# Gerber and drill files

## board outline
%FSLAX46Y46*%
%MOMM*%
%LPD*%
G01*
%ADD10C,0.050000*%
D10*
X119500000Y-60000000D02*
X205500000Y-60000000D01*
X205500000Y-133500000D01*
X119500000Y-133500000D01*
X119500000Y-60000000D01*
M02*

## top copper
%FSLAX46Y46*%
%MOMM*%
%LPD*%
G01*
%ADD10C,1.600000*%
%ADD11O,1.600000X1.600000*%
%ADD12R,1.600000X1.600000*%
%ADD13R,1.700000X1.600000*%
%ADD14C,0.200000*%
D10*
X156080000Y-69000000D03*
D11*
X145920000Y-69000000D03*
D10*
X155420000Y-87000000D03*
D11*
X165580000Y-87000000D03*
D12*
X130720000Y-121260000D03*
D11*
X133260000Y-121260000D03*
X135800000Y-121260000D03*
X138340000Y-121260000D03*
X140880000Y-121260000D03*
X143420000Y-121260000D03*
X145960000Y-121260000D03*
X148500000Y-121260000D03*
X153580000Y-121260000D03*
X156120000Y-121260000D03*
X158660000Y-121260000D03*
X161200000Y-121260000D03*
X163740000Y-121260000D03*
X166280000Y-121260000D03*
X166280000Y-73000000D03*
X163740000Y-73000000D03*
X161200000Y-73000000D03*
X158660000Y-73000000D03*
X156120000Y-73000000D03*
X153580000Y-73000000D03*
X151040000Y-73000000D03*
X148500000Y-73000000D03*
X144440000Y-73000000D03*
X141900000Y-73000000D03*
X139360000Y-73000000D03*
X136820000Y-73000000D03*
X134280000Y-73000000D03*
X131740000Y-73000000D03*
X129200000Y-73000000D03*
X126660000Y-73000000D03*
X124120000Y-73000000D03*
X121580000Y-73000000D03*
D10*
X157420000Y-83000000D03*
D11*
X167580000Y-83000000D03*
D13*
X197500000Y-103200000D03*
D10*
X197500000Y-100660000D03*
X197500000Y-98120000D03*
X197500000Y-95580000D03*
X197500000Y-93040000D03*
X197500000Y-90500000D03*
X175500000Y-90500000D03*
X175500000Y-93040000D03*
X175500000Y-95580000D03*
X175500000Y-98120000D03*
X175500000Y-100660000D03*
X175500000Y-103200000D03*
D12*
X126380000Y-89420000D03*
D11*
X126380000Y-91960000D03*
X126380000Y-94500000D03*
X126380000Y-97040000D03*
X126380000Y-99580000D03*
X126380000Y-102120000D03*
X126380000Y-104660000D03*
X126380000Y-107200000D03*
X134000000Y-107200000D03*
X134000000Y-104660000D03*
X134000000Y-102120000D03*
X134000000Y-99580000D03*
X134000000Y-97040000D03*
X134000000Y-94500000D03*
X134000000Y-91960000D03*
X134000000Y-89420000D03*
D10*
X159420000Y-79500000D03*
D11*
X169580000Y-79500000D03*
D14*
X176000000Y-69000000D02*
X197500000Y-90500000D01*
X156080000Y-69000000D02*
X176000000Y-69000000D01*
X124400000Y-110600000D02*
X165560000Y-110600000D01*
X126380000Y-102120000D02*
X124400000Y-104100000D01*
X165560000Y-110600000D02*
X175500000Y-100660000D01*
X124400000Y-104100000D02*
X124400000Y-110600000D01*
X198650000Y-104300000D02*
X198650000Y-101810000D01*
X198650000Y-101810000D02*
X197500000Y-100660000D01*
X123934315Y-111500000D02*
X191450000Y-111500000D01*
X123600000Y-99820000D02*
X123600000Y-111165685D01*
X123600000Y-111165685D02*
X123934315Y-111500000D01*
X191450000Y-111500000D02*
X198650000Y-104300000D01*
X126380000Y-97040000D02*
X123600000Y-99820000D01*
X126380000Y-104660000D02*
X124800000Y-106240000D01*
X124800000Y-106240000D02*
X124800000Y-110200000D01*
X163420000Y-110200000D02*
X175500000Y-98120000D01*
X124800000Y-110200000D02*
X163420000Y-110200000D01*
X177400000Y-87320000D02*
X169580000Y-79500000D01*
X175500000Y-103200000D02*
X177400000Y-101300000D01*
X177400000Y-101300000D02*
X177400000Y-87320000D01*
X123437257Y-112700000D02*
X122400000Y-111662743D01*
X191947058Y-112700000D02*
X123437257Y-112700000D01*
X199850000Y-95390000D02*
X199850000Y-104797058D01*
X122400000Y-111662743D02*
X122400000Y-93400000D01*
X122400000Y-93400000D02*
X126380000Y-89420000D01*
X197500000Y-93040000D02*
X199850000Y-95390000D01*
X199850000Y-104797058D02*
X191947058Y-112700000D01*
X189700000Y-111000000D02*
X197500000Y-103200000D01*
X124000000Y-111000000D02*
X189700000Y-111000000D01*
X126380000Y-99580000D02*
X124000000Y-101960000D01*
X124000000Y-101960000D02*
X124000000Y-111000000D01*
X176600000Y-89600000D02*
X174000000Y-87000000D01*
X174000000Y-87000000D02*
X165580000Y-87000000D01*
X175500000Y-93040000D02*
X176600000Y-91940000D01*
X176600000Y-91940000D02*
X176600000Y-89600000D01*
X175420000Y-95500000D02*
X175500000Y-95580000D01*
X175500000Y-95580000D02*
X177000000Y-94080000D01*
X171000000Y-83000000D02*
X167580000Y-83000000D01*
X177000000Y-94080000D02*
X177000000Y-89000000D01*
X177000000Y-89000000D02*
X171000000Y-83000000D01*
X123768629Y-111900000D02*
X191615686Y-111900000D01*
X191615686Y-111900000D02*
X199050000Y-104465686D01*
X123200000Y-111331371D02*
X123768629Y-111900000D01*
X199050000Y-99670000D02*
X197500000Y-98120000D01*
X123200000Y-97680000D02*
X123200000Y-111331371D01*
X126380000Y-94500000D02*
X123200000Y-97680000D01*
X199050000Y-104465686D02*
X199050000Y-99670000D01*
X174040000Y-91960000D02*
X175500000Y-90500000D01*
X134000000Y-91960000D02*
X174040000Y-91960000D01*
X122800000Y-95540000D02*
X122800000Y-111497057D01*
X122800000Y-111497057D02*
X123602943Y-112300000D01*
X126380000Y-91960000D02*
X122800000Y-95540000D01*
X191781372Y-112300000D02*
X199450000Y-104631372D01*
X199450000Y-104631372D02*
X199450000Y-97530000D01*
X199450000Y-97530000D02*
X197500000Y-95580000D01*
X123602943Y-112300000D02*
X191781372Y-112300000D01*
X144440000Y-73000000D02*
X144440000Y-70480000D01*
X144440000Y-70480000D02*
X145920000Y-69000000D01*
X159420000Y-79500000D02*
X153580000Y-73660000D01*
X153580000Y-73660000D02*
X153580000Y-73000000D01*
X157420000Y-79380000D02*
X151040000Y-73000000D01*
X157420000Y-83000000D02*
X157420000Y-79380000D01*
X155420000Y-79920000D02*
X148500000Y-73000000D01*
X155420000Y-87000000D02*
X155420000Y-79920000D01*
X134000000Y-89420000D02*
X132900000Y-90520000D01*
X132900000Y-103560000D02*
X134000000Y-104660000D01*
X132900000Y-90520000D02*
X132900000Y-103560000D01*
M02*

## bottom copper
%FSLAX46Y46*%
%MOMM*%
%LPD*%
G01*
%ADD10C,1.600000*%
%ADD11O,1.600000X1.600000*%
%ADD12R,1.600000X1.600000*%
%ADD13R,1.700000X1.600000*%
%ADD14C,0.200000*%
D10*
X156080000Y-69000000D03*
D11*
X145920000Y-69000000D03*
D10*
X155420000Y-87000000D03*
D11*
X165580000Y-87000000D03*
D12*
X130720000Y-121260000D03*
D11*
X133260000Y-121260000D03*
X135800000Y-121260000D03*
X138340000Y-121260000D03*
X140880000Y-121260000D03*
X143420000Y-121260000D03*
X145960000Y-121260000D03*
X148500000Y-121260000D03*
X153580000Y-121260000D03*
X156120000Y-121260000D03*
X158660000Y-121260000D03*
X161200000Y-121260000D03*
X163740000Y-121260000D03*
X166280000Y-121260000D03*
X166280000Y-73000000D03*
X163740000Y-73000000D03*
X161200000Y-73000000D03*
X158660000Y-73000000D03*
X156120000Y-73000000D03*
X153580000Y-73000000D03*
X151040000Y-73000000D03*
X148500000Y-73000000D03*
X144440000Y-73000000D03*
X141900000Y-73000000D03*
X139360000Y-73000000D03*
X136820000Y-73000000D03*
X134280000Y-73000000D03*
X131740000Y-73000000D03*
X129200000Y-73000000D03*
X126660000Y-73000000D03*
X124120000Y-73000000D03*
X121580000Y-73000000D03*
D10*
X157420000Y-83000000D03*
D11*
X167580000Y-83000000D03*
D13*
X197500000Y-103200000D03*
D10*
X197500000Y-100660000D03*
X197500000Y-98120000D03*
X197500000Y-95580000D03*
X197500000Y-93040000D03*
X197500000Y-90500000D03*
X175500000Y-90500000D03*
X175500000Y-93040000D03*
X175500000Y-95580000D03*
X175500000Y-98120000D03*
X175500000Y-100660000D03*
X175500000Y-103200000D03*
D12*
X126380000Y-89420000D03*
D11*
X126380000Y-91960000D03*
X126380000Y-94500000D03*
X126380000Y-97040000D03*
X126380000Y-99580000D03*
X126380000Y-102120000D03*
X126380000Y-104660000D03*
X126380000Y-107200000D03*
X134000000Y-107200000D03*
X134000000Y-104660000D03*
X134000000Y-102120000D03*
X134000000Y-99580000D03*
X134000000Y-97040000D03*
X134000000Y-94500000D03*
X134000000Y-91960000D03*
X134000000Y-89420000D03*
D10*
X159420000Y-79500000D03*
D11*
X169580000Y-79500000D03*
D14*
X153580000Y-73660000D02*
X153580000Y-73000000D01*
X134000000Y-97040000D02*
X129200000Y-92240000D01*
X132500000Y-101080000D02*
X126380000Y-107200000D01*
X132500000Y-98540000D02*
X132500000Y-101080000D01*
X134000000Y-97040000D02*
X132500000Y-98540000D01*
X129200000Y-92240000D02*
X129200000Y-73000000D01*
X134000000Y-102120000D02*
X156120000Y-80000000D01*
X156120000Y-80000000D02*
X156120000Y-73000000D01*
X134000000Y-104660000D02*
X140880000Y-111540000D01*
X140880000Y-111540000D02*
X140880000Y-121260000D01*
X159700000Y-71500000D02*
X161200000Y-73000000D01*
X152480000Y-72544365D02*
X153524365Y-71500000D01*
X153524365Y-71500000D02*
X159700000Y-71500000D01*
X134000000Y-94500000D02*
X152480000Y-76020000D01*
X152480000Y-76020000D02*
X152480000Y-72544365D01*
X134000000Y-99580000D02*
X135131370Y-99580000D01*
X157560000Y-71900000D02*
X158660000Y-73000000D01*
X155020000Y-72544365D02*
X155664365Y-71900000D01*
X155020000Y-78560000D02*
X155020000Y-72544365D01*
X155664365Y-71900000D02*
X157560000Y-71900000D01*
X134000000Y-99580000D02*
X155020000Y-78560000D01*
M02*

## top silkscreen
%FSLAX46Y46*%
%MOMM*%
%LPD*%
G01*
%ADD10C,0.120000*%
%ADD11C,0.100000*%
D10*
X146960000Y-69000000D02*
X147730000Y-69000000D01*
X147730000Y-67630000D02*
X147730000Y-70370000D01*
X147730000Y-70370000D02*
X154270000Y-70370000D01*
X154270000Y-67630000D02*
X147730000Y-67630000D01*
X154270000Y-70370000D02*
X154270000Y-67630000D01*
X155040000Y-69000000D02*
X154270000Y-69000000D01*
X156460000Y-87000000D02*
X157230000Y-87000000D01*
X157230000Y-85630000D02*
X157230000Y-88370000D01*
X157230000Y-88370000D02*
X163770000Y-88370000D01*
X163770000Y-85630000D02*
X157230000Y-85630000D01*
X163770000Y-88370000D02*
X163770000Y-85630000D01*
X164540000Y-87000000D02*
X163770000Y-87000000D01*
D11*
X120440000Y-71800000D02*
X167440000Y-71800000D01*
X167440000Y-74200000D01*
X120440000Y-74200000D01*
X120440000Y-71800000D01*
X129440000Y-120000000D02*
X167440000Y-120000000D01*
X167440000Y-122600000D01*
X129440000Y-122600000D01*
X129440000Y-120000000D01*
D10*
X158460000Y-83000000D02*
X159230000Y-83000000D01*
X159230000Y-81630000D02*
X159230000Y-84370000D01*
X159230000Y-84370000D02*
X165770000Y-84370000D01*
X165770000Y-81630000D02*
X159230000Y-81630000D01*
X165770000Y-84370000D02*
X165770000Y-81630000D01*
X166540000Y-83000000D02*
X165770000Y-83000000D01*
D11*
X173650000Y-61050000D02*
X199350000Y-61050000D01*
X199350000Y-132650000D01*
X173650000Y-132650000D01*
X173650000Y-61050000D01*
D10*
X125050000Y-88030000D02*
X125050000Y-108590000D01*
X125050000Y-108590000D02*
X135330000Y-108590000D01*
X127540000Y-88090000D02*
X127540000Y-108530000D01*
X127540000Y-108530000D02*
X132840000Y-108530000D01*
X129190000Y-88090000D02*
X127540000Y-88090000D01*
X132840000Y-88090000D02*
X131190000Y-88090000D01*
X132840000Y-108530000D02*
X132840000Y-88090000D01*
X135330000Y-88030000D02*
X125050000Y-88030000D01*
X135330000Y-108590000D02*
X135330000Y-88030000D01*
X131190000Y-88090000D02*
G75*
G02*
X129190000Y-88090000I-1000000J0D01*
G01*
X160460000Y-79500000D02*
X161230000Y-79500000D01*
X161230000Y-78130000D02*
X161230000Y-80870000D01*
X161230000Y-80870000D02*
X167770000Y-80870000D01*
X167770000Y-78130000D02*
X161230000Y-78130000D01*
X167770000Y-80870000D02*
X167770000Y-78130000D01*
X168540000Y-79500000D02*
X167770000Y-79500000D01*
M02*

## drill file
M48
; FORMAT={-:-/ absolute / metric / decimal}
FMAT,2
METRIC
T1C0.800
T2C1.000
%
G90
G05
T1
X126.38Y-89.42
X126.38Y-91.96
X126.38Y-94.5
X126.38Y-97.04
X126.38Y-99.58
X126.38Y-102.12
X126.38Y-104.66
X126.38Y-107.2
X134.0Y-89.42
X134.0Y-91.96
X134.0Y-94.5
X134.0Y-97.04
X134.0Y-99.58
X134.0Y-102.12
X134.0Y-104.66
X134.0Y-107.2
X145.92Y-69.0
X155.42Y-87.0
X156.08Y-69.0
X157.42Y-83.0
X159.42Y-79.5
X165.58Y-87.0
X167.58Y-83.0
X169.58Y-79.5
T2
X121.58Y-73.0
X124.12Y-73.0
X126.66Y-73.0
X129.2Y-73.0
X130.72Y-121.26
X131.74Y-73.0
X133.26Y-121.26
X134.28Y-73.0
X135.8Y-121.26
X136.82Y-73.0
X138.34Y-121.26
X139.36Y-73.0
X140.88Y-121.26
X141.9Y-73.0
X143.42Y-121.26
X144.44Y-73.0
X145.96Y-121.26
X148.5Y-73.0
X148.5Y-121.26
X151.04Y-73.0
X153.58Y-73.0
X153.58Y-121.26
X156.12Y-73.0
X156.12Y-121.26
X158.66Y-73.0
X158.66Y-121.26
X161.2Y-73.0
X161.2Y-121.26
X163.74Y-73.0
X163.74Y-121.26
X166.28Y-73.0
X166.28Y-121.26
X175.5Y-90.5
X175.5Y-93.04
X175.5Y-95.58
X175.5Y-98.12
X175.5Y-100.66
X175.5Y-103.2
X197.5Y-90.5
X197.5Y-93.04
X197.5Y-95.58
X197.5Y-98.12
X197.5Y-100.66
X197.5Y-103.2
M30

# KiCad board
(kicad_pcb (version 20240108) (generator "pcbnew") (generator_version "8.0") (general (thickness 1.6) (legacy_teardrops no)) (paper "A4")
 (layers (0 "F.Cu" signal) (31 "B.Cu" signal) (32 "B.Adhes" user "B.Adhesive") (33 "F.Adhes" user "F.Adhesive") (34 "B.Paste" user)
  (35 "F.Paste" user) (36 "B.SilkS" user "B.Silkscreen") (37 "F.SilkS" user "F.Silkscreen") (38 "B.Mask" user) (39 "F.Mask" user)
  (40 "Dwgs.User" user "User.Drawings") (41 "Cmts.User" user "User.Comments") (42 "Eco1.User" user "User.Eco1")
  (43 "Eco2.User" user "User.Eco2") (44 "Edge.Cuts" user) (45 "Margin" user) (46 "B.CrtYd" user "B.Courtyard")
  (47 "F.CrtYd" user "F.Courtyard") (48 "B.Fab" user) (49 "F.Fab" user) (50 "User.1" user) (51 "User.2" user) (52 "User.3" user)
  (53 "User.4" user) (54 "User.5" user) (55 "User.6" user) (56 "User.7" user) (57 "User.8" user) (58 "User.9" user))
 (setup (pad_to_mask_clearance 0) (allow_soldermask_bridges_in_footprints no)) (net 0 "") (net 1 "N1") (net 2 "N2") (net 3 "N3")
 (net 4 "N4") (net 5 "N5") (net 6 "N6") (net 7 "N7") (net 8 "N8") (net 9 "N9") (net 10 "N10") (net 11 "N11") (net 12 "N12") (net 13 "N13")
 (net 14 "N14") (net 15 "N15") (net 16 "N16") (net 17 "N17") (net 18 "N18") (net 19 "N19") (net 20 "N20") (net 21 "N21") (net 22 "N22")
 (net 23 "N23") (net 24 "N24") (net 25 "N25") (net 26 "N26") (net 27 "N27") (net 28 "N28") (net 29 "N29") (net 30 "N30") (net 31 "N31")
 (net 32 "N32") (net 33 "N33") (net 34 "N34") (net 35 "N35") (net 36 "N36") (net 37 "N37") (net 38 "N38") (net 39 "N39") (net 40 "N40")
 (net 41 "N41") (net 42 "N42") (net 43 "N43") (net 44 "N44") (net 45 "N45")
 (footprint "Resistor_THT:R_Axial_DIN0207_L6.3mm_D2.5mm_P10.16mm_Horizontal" (layer "F.Cu") (at 156.08 69 180)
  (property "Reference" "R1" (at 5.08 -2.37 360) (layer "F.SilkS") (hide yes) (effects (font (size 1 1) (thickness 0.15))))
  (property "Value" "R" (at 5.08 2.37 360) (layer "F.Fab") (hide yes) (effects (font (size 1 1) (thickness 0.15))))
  (fp_line (start 9.12 0) (end 8.35 0) (stroke (width 0.12) (type solid)) (layer "F.SilkS"))
  (fp_line (start 8.35 1.37) (end 8.35 -1.37) (stroke (width 0.12) (type solid)) (layer "F.SilkS"))
  (fp_line (start 8.35 -1.37) (end 1.81 -1.37) (stroke (width 0.12) (type solid)) (layer "F.SilkS"))
  (fp_line (start 1.81 1.37) (end 8.35 1.37) (stroke (width 0.12) (type solid)) (layer "F.SilkS"))
  (fp_line (start 1.81 -1.37) (end 1.81 1.37) (stroke (width 0.12) (type solid)) (layer "F.SilkS"))
  (fp_line (start 1.04 0) (end 1.81 0) (stroke (width 0.12) (type solid)) (layer "F.SilkS"))
  (pad "1" thru_hole circle (at 0 0 180) (size 1.6 1.6) (drill 0.8) (layers "*.Cu" "*.Mask") (remove_unused_layers no) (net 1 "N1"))
  (pad "2" thru_hole oval (at 10.16 0 180) (size 1.6 1.6) (drill 0.8) (layers "*.Cu" "*.Mask") (remove_unused_layers no) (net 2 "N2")))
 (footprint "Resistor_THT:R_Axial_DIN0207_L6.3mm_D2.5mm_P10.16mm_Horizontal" (layer "F.Cu") (at 155.42 87)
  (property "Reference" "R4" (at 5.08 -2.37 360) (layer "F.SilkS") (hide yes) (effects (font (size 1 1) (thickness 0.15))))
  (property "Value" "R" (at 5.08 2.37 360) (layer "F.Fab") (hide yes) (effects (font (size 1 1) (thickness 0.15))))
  (fp_line (start 1.04 0) (end 1.81 0) (stroke (width 0.12) (type solid)) (layer "F.SilkS"))
  (fp_line (start 1.81 -1.37) (end 1.81 1.37) (stroke (width 0.12) (type solid)) (layer "F.SilkS"))
  (fp_line (start 1.81 1.37) (end 8.35 1.37) (stroke (width 0.12) (type solid)) (layer "F.SilkS"))
  (fp_line (start 8.35 -1.37) (end 1.81 -1.37) (stroke (width 0.12) (type solid)) (layer "F.SilkS"))
  (fp_line (start 8.35 1.37) (end 8.35 -1.37) (stroke (width 0.12) (type solid)) (layer "F.SilkS"))
  (fp_line (start 9.12 0) (end 8.35 0) (stroke (width 0.12) (type solid)) (layer "F.SilkS"))
  (pad "1" thru_hole circle (at 0 0) (size 1.6 1.6) (drill 0.8) (layers "*.Cu" "*.Mask") (remove_unused_layers no) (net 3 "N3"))
  (pad "2" thru_hole oval (at 10.16 0) (size 1.6 1.6) (drill 0.8) (layers "*.Cu" "*.Mask") (remove_unused_layers no) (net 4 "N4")))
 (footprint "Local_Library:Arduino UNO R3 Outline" (layer "F.Cu") (at 109.84 75.2)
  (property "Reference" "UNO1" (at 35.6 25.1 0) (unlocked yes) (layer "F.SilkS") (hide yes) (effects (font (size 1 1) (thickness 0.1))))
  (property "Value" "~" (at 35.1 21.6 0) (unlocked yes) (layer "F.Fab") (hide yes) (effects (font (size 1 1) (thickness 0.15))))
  (fp_rect (start 10.6 -3.4) (end 57.6 -1) (stroke (width 0.1) (type default)) (fill none) (layer "F.SilkS"))
  (fp_rect (start 19.6 44.8) (end 57.6 47.4) (stroke (width 0.1) (type default)) (fill none) (layer "F.SilkS"))
  (pad "1" thru_hole rect (at 20.88 46.06 90) (size 1.6 1.6) (drill 1) (layers "*.Cu" "*.Mask") (remove_unused_layers no) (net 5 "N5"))
  (pad "2" thru_hole oval (at 23.42 46.06 90) (size 1.6 1.6) (drill 1) (layers "*.Cu" "*.Mask") (remove_unused_layers no) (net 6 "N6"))
  (pad "3" thru_hole oval (at 25.96 46.06 90) (size 1.6 1.6) (drill 1) (layers "*.Cu" "*.Mask") (remove_unused_layers no) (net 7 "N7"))
  (pad "4" thru_hole oval (at 28.5 46.06 90) (size 1.6 1.6) (drill 1) (layers "*.Cu" "*.Mask") (remove_unused_layers no) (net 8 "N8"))
  (pad "5" thru_hole oval (at 31.04 46.06 90) (size 1.6 1.6) (drill 1) (layers "*.Cu" "*.Mask") (remove_unused_layers no) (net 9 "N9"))
  (pad "6" thru_hole oval (at 33.58 46.06 90) (size 1.6 1.6) (drill 1) (layers "*.Cu" "*.Mask") (remove_unused_layers no) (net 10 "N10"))
  (pad "7" thru_hole oval (at 36.12 46.06 90) (size 1.6 1.6) (drill 1) (layers "*.Cu" "*.Mask") (remove_unused_layers no) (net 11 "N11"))
  (pad "8" thru_hole oval (at 38.66 46.06 90) (size 1.6 1.6) (drill 1) (layers "*.Cu" "*.Mask") (remove_unused_layers no) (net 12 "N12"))
  (pad "9" thru_hole oval (at 43.74 46.06 90) (size 1.6 1.6) (drill 1) (layers "*.Cu" "*.Mask") (remove_unused_layers no) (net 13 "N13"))
  (pad "10" thru_hole oval (at 46.28 46.06 90) (size 1.6 1.6) (drill 1) (layers "*.Cu" "*.Mask") (remove_unused_layers no) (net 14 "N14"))
  (pad "11" thru_hole oval (at 48.82 46.06 90) (size 1.6 1.6) (drill 1) (layers "*.Cu" "*.Mask") (remove_unused_layers no) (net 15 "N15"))
  (pad "12" thru_hole oval (at 51.36 46.06 90) (size 1.6 1.6) (drill 1) (layers "*.Cu" "*.Mask") (remove_unused_layers no) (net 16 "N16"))
  (pad "13" thru_hole oval (at 53.9 46.06 90) (size 1.6 1.6) (drill 1) (layers "*.Cu" "*.Mask") (remove_unused_layers no) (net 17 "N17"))
  (pad "14" thru_hole oval (at 56.44 46.06 90) (size 1.6 1.6) (drill 1) (layers "*.Cu" "*.Mask") (remove_unused_layers no) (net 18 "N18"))
  (pad "15" thru_hole oval (at 56.44 -2.2 90) (size 1.6 1.6) (drill 1) (layers "*.Cu" "*.Mask") (remove_unused_layers no) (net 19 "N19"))
  (pad "16" thru_hole oval (at 53.9 -2.2 90) (size 1.6 1.6) (drill 1) (layers "*.Cu" "*.Mask") (remove_unused_layers no) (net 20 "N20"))
  (pad "17" thru_hole oval (at 51.36 -2.2 90) (size 1.6 1.6) (drill 1) (layers "*.Cu" "*.Mask") (remove_unused_layers no) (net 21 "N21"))
  (pad "18" thru_hole oval (at 48.82 -2.2 90) (size 1.6 1.6) (drill 1) (layers "*.Cu" "*.Mask") (remove_unused_layers no) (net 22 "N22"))
  (pad "19" thru_hole oval (at 46.28 -2.2 90) (size 1.6 1.6) (drill 1) (layers "*.Cu" "*.Mask") (remove_unused_layers no) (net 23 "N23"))
  (pad "20" thru_hole oval (at 43.74 -2.2 90) (size 1.6 1.6) (drill 1) (layers "*.Cu" "*.Mask") (remove_unused_layers no) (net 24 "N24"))
  (pad "21" thru_hole oval (at 41.2 -2.2 90) (size 1.6 1.6) (drill 1) (layers "*.Cu" "*.Mask") (remove_unused_layers no) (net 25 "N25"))
  (pad "22" thru_hole oval (at 38.66 -2.2 90) (size 1.6 1.6) (drill 1) (layers "*.Cu" "*.Mask") (remove_unused_layers no) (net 3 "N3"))
  (pad "23" thru_hole oval (at 34.6 -2.2 90) (size 1.6 1.6) (drill 1) (layers "*.Cu" "*.Mask") (remove_unused_layers no) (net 2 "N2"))
  (pad "24" thru_hole oval (at 32.06 -2.2 90) (size 1.6 1.6) (drill 1) (layers "*.Cu" "*.Mask") (remove_unused_layers no) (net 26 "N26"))
  (pad "25" thru_hole oval (at 29.52 -2.2 90) (size 1.6 1.6) (drill 1) (layers "*.Cu" "*.Mask") (remove_unused_layers no) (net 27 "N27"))
  (pad "26" thru_hole oval (at 26.98 -2.2 90) (size 1.6 1.6) (drill 1) (layers "*.Cu" "*.Mask") (remove_unused_layers no) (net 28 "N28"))
  (pad "27" thru_hole oval (at 24.44 -2.2 90) (size 1.6 1.6) (drill 1) (layers "*.Cu" "*.Mask") (remove_unused_layers no) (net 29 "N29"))
  (pad "28" thru_hole oval (at 21.9 -2.2 90) (size 1.6 1.6) (drill 1) (layers "*.Cu" "*.Mask") (remove_unused_layers no) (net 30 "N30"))
  (pad "29" thru_hole oval (at 19.36 -2.2 90) (size 1.6 1.6) (drill 1) (layers "*.Cu" "*.Mask") (remove_unused_layers no) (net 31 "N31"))
  (pad "30" thru_hole oval (at 16.82 -2.2 90) (size 1.6 1.6) (drill 1) (layers "*.Cu" "*.Mask") (remove_unused_layers no) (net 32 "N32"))
  (pad "31" thru_hole oval (at 14.28 -2.2 90) (size 1.6 1.6) (drill 1) (layers "*.Cu" "*.Mask") (remove_unused_layers no) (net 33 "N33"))
  (pad "32" thru_hole oval (at 11.74 -2.2 90) (size 1.6 1.6) (drill 1) (layers "*.Cu" "*.Mask") (remove_unused_layers no) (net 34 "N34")))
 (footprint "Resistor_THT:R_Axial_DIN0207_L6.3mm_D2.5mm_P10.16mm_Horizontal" (layer "F.Cu") (at 157.42 83)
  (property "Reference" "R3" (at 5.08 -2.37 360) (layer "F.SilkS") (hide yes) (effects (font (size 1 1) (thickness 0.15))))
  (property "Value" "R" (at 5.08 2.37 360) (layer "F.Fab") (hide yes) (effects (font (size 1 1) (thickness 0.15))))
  (fp_line (start 1.04 0) (end 1.81 0) (stroke (width 0.12) (type solid)) (layer "F.SilkS"))
  (fp_line (start 1.81 -1.37) (end 1.81 1.37) (stroke (width 0.12) (type solid)) (layer "F.SilkS"))
  (fp_line (start 1.81 1.37) (end 8.35 1.37) (stroke (width 0.12) (type solid)) (layer "F.SilkS"))
  (fp_line (start 8.35 -1.37) (end 1.81 -1.37) (stroke (width 0.12) (type solid)) (layer "F.SilkS"))
  (fp_line (start 8.35 1.37) (end 8.35 -1.37) (stroke (width 0.12) (type solid)) (layer "F.SilkS"))
  (fp_line (start 9.12 0) (end 8.35 0) (stroke (width 0.12) (type solid)) (layer "F.SilkS"))
  (pad "1" thru_hole circle (at 0 0) (size 1.6 1.6) (drill 0.8) (layers "*.Cu" "*.Mask") (remove_unused_layers no) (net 25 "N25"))
  (pad "2" thru_hole oval (at 10.16 0) (size 1.6 1.6) (drill 0.8) (layers "*.Cu" "*.Mask") (remove_unused_layers no) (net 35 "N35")))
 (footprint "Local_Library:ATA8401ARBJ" (layer "F.Cu") (at 186.5 96.85 90)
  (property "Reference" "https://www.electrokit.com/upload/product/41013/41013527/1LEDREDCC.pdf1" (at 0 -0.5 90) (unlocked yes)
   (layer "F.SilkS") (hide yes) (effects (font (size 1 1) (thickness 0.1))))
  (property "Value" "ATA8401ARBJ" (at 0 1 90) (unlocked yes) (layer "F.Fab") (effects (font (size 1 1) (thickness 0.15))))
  (fp_rect (start -35.8 -12.85) (end 35.8 12.85) (stroke (width 0.1) (type default)) (fill none) (layer "F.SilkS"))
  (pad "1" thru_hole rect (at -6.35 11 90) (size 1.6 1.7) (drill 1) (layers "*.Cu" "*.Mask") (remove_unused_layers no) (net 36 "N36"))
  (pad "2" thru_hole circle (at -3.81 11 90) (size 1.6 1.6) (drill 1) (layers "*.Cu" "*.Mask") (remove_unused_layers no) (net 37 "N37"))
  (pad "3" thru_hole circle (at -1.27 11 90) (size 1.6 1.6) (drill 1) (layers "*.Cu" "*.Mask") (remove_unused_layers no) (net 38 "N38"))
  (pad "4" thru_hole circle (at 1.27 11 90) (size 1.6 1.6) (drill 1) (layers "*.Cu" "*.Mask") (remove_unused_layers no) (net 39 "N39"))
  (pad "5" thru_hole circle (at 3.81 11 90) (size 1.6 1.6) (drill 1) (layers "*.Cu" "*.Mask") (remove_unused_layers no) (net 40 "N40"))
  (pad "6" thru_hole circle (at 6.35 11 90) (size 1.6 1.6) (drill 1) (layers "*.Cu" "*.Mask") (remove_unused_layers no) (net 1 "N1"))
  (pad "7" thru_hole circle (at 6.35 -11 270) (size 1.6 1.6) (drill 1) (layers "*.Cu" "*.Mask") (remove_unused_layers no) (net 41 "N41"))
  (pad "8" thru_hole circle (at 3.81 -11 270) (size 1.6 1.6) (drill 1) (layers "*.Cu" "*.Mask") (remove_unused_layers no) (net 4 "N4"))
  (pad "9" thru_hole circle (at 1.27 -11 270) (size 1.6 1.6) (drill 1) (layers "*.Cu" "*.Mask") (remove_unused_layers no) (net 35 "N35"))
  (pad "10" thru_hole circle (at -1.27 -11 270) (size 1.6 1.6) (drill 1) (layers "*.Cu" "*.Mask") (remove_unused_layers no) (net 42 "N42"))
  (pad "11" thru_hole circle (at -3.81 -11 270) (size 1.6 1.6) (drill 1) (layers "*.Cu" "*.Mask") (remove_unused_layers no) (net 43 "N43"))
  (pad "12" thru_hole circle (at -6.35 -11 270) (size 1.6 1.6) (drill 1) (layers "*.Cu" "*.Mask") (remove_unused_layers no) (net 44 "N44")))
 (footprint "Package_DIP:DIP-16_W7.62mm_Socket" (layer "F.Cu") (at 126.38 89.42)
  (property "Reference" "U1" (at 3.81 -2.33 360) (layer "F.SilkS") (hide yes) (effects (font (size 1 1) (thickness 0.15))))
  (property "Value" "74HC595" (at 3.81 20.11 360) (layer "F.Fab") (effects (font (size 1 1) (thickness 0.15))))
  (fp_line (start -1.33 -1.39) (end -1.33 19.17) (stroke (width 0.12) (type solid)) (layer "F.SilkS"))
  (fp_line (start -1.33 19.17) (end 8.95 19.17) (stroke (width 0.12) (type solid)) (layer "F.SilkS"))
  (fp_line (start 1.16 -1.33) (end 1.16 19.11) (stroke (width 0.12) (type solid)) (layer "F.SilkS"))
  (fp_line (start 1.16 19.11) (end 6.46 19.11) (stroke (width 0.12) (type solid)) (layer "F.SilkS"))
  (fp_line (start 2.81 -1.33) (end 1.16 -1.33) (stroke (width 0.12) (type solid)) (layer "F.SilkS"))
  (fp_line (start 6.46 -1.33) (end 4.81 -1.33) (stroke (width 0.12) (type solid)) (layer "F.SilkS"))
  (fp_line (start 6.46 19.11) (end 6.46 -1.33) (stroke (width 0.12) (type solid)) (layer "F.SilkS"))
  (fp_line (start 8.95 -1.39) (end -1.33 -1.39) (stroke (width 0.12) (type solid)) (layer "F.SilkS"))
  (fp_line (start 8.95 19.17) (end 8.95 -1.39) (stroke (width 0.12) (type solid)) (layer "F.SilkS"))
  (fp_arc (start 4.81 -1.33) (mid 3.81 -0.33) (end 2.81 -1.33) (stroke (width 0.12) (type solid)) (layer "F.SilkS"))
  (pad "1" thru_hole rect (at 0 0) (size 1.6 1.6) (drill 0.8) (layers "*.Cu" "*.Mask") (remove_unused_layers no) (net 40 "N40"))
  (pad "2" thru_hole oval (at 0 2.54) (size 1.6 1.6) (drill 0.8) (layers "*.Cu" "*.Mask") (remove_unused_layers no) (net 39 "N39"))
  (pad "3" thru_hole oval (at 0 5.08) (size 1.6 1.6) (drill 0.8) (layers "*.Cu" "*.Mask") (remove_unused_layers no) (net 38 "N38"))
  (pad "4" thru_hole oval (at 0 7.62) (size 1.6 1.6) (drill 0.8) (layers "*.Cu" "*.Mask") (remove_unused_layers no) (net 37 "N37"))
  (pad "5" thru_hole oval (at 0 10.16) (size 1.6 1.6) (drill 0.8) (layers "*.Cu" "*.Mask") (remove_unused_layers no) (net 36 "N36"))
  (pad "6" thru_hole oval (at 0 12.7) (size 1.6 1.6) (drill 0.8) (layers "*.Cu" "*.Mask") (remove_unused_layers no) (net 43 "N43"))
  (pad "7" thru_hole oval (at 0 15.24) (size 1.6 1.6) (drill 0.8) (layers "*.Cu" "*.Mask") (remove_unused_layers no) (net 42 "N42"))
  (pad "8" thru_hole oval (at 0 17.78) (size 1.6 1.6) (drill 0.8) (layers "*.Cu" "*.Mask") (remove_unused_layers no) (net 31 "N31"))
  (pad "9" thru_hole oval (at 7.62 17.78) (size 1.6 1.6) (drill 0.8) (layers "*.Cu" "*.Mask") (remove_unused_layers no) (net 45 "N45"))
  (pad "10" thru_hole oval (at 7.62 15.24) (size 1.6 1.6) (drill 0.8) (layers "*.Cu" "*.Mask") (remove_unused_layers no) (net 9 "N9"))
  (pad "11" thru_hole oval (at 7.62 12.7) (size 1.6 1.6) (drill 0.8) (layers "*.Cu" "*.Mask") (remove_unused_layers no) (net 23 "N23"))
  (pad "12" thru_hole oval (at 7.62 10.16) (size 1.6 1.6) (drill 0.8) (layers "*.Cu" "*.Mask") (remove_unused_layers no) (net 22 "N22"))
  (pad "13" thru_hole oval (at 7.62 7.62) (size 1.6 1.6) (drill 0.8) (layers "*.Cu" "*.Mask") (remove_unused_layers no) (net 31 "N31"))
  (pad "14" thru_hole oval (at 7.62 5.08) (size 1.6 1.6) (drill 0.8) (layers "*.Cu" "*.Mask") (remove_unused_layers no) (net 21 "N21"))
  (pad "15" thru_hole oval (at 7.62 2.54) (size 1.6 1.6) (drill 0.8) (layers "*.Cu" "*.Mask") (remove_unused_layers no) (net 41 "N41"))
  (pad "16" thru_hole oval (at 7.62 0) (size 1.6 1.6) (drill 0.8) (layers "*.Cu" "*.Mask") (remove_unused_layers no) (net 9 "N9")))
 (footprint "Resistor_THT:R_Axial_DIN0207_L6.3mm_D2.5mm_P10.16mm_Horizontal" (layer "F.Cu") (at 159.42 79.5)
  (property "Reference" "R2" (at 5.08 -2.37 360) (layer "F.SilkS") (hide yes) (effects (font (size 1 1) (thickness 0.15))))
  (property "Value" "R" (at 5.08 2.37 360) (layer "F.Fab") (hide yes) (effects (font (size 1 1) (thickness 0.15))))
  (fp_line (start 1.04 0) (end 1.81 0) (stroke (width 0.12) (type solid)) (layer "F.SilkS"))
  (fp_line (start 1.81 -1.37) (end 1.81 1.37) (stroke (width 0.12) (type solid)) (layer "F.SilkS"))
  (fp_line (start 1.81 1.37) (end 8.35 1.37) (stroke (width 0.12) (type solid)) (layer "F.SilkS"))
  (fp_line (start 8.35 -1.37) (end 1.81 -1.37) (stroke (width 0.12) (type solid)) (layer "F.SilkS"))
  (fp_line (start 8.35 1.37) (end 8.35 -1.37) (stroke (width 0.12) (type solid)) (layer "F.SilkS"))
  (fp_line (start 9.12 0) (end 8.35 0) (stroke (width 0.12) (type solid)) (layer "F.SilkS"))
  (pad "1" thru_hole circle (at 0 0) (size 1.6 1.6) (drill 0.8) (layers "*.Cu" "*.Mask") (remove_unused_layers no) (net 24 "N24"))
  (pad "2" thru_hole oval (at 10.16 0) (size 1.6 1.6) (drill 0.8) (layers "*.Cu" "*.Mask") (remove_unused_layers no) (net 44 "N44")))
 (gr_rect (start 119.5 60) (end 205.5 133.5) (stroke (width 0.05) (type default)) (fill none) (layer "Edge.Cuts"))
 (segment (start 176 69) (end 197.5 90.5) (width 0.2) (layer "F.Cu") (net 1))
 (segment (start 156.08 69) (end 176 69) (width 0.2) (layer "F.Cu") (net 1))
 (segment (start 124.4 110.6) (end 165.56 110.6) (width 0.2) (layer "F.Cu") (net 43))
 (segment (start 126.38 102.12) (end 124.4 104.1) (width 0.2) (layer "F.Cu") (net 43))
 (segment (start 165.56 110.6) (end 175.5 100.66) (width 0.2) (layer "F.Cu") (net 43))
 (segment (start 124.4 104.1) (end 124.4 110.6) (width 0.2) (layer "F.Cu") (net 43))
 (segment (start 198.65 104.3) (end 198.65 101.81) (width 0.2) (layer "F.Cu") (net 37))
 (segment (start 198.65 101.81) (end 197.5 100.66) (width 0.2) (layer "F.Cu") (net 37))
 (segment (start 123.934315 111.5) (end 191.45 111.5) (width 0.2) (layer "F.Cu") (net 37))
 (segment (start 123.6 99.82) (end 123.6 111.165685) (width 0.2) (layer "F.Cu") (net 37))
 (segment (start 123.6 111.165685) (end 123.934315 111.5) (width 0.2) (layer "F.Cu") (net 37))
 (segment (start 191.45 111.5) (end 198.65 104.3) (width 0.2) (layer "F.Cu") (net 37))
 (segment (start 126.38 97.04) (end 123.6 99.82) (width 0.2) (layer "F.Cu") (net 37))
 (segment (start 126.38 104.66) (end 124.8 106.24) (width 0.2) (layer "F.Cu") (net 42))
 (segment (start 124.8 106.24) (end 124.8 110.2) (width 0.2) (layer "F.Cu") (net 42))
 (segment (start 163.42 110.2) (end 175.5 98.12) (width 0.2) (layer "F.Cu") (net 42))
 (segment (start 124.8 110.2) (end 163.42 110.2) (width 0.2) (layer "F.Cu") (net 42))
 (segment (start 177.4 87.32) (end 169.58 79.5) (width 0.2) (layer "F.Cu") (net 44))
 (segment (start 175.5 103.2) (end 177.4 101.3) (width 0.2) (layer "F.Cu") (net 44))
 (segment (start 177.4 101.3) (end 177.4 87.32) (width 0.2) (layer "F.Cu") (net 44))
 (segment (start 123.437257 112.7) (end 122.4 111.662743) (width 0.2) (layer "F.Cu") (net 40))
 (segment (start 191.947058 112.7) (end 123.437257 112.7) (width 0.2) (layer "F.Cu") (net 40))
 (segment (start 199.85 95.39) (end 199.85 104.797058) (width 0.2) (layer "F.Cu") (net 40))
 (segment (start 122.4 111.662743) (end 122.4 93.4) (width 0.2) (layer "F.Cu") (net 40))
 (segment (start 122.4 93.4) (end 126.38 89.42) (width 0.2) (layer "F.Cu") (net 40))
 (segment (start 197.5 93.04) (end 199.85 95.39) (width 0.2) (layer "F.Cu") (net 40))
 (segment (start 199.85 104.797058) (end 191.947058 112.7) (width 0.2) (layer "F.Cu") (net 40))
 (segment (start 189.7 111) (end 197.5 103.2) (width 0.2) (layer "F.Cu") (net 36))
 (segment (start 124 111) (end 189.7 111) (width 0.2) (layer "F.Cu") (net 36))
 (segment (start 126.38 99.58) (end 124 101.96) (width 0.2) (layer "F.Cu") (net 36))
 (segment (start 124 101.96) (end 124 111) (width 0.2) (layer "F.Cu") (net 36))
 (segment (start 176.6 89.6) (end 174 87) (width 0.2) (layer "F.Cu") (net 4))
 (segment (start 174 87) (end 165.58 87) (width 0.2) (layer "F.Cu") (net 4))
 (segment (start 175.5 93.04) (end 176.6 91.94) (width 0.2) (layer "F.Cu") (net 4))
 (segment (start 176.6 91.94) (end 176.6 89.6) (width 0.2) (layer "F.Cu") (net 4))
 (segment (start 175.42 95.5) (end 175.5 95.58) (width 0.2) (layer "F.Cu") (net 35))
 (segment (start 175.5 95.58) (end 177 94.08) (width 0.2) (layer "F.Cu") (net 35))
 (segment (start 171 83) (end 167.58 83) (width 0.2) (layer "F.Cu") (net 35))
 (segment (start 177 94.08) (end 177 89) (width 0.2) (layer "F.Cu") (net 35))
 (segment (start 177 89) (end 171 83) (width 0.2) (layer "F.Cu") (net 35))
 (segment (start 123.768629 111.9) (end 191.615686 111.9) (width 0.2) (layer "F.Cu") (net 38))
 (segment (start 191.615686 111.9) (end 199.05 104.465686) (width 0.2) (layer "F.Cu") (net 38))
 (segment (start 123.2 111.331371) (end 123.768629 111.9) (width 0.2) (layer "F.Cu") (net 38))
 (segment (start 199.05 99.67) (end 197.5 98.12) (width 0.2) (layer "F.Cu") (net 38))
 (segment (start 123.2 97.68) (end 123.2 111.331371) (width 0.2) (layer "F.Cu") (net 38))
 (segment (start 126.38 94.5) (end 123.2 97.68) (width 0.2) (layer "F.Cu") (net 38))
 (segment (start 199.05 104.465686) (end 199.05 99.67) (width 0.2) (layer "F.Cu") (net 38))
 (segment (start 174.04 91.96) (end 175.5 90.5) (width 0.2) (layer "F.Cu") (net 41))
 (segment (start 134 91.96) (end 174.04 91.96) (width 0.2) (layer "F.Cu") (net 41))
 (segment (start 122.8 95.54) (end 122.8 111.497057) (width 0.2) (layer "F.Cu") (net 39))
 (segment (start 122.8 111.497057) (end 123.602943 112.3) (width 0.2) (layer "F.Cu") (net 39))
 (segment (start 126.38 91.96) (end 122.8 95.54) (width 0.2) (layer "F.Cu") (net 39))
 (segment (start 191.781372 112.3) (end 199.45 104.631372) (width 0.2) (layer "F.Cu") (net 39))
 (segment (start 199.45 104.631372) (end 199.45 97.53) (width 0.2) (layer "F.Cu") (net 39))
 (segment (start 199.45 97.53) (end 197.5 95.58) (width 0.2) (layer "F.Cu") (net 39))
 (segment (start 123.602943 112.3) (end 191.781372 112.3) (width 0.2) (layer "F.Cu") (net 39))
 (segment (start 144.44 73) (end 144.44 70.48) (width 0.2) (layer "F.Cu") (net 2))
 (segment (start 144.44 70.48) (end 145.92 69) (width 0.2) (layer "F.Cu") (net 2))
 (segment (start 159.42 79.5) (end 153.58 73.66) (width 0.2) (layer "F.Cu") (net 24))
 (segment (start 153.58 73.66) (end 153.58 73) (width 0.2) (layer "F.Cu") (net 24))
 (segment (start 153.58 73.66) (end 153.58 73) (width 0.2) (layer "B.Cu") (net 24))
 (segment (start 157.42 79.38) (end 151.04 73) (width 0.2) (layer "F.Cu") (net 25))
 (segment (start 157.42 83) (end 157.42 79.38) (width 0.2) (layer "F.Cu") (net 25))
 (segment (start 155.42 79.92) (end 148.5 73) (width 0.2) (layer "F.Cu") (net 3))
 (segment (start 155.42 87) (end 155.42 79.92) (width 0.2) (layer "F.Cu") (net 3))
 (segment (start 134 97.04) (end 129.2 92.24) (width 0.2) (layer "B.Cu") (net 31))
 (segment (start 132.5 101.08) (end 126.38 107.2) (width 0.2) (layer "B.Cu") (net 31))
 (segment (start 132.5 98.54) (end 132.5 101.08) (width 0.2) (layer "B.Cu") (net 31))
 (segment (start 134 97.04) (end 132.5 98.54) (width 0.2) (layer "B.Cu") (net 31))
 (segment (start 129.2 92.24) (end 129.2 73) (width 0.2) (layer "B.Cu") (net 31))
 (segment (start 134 102.12) (end 156.12 80) (width 0.2) (layer "B.Cu") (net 23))
 (segment (start 156.12 80) (end 156.12 73) (width 0.2) (layer "B.Cu") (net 23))
 (segment (start 134 89.42) (end 132.9 90.52) (width 0.2) (layer "F.Cu") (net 9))
 (segment (start 132.9 103.56) (end 134 104.66) (width 0.2) (layer "F.Cu") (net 9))
 (segment (start 132.9 90.52) (end 132.9 103.56) (width 0.2) (layer "F.Cu") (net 9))
 (segment (start 134 104.66) (end 140.88 111.54) (width 0.2) (layer "B.Cu") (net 9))
 (segment (start 140.88 111.54) (end 140.88 121.26) (width 0.2) (layer "B.Cu") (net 9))
 (segment (start 159.7 71.5) (end 161.2 73) (width 0.2) (layer "B.Cu") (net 21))
 (segment (start 152.48 72.544365) (end 153.524365 71.5) (width 0.2) (layer "B.Cu") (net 21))
 (segment (start 153.524365 71.5) (end 159.7 71.5) (width 0.2) (layer "B.Cu") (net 21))
 (segment (start 134 94.5) (end 152.48 76.02) (width 0.2) (layer "B.Cu") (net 21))
 (segment (start 152.48 76.02) (end 152.48 72.544365) (width 0.2) (layer "B.Cu") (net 21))
 (segment (start 134 99.58) (end 135.13137 99.58) (width 0.2) (layer "B.Cu") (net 22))
 (segment (start 157.56 71.9) (end 158.66 73) (width 0.2) (layer "B.Cu") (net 22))
 (segment (start 155.02 72.544365) (end 155.664365 71.9) (width 0.2) (layer "B.Cu") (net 22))
 (segment (start 155.02 78.56) (end 155.02 72.544365) (width 0.2) (layer "B.Cu") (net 22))
 (segment (start 155.664365 71.9) (end 157.56 71.9) (width 0.2) (layer "B.Cu") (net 22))
 (segment (start 134 99.58) (end 155.02 78.56) (width 0.2) (layer "B.Cu") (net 22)))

